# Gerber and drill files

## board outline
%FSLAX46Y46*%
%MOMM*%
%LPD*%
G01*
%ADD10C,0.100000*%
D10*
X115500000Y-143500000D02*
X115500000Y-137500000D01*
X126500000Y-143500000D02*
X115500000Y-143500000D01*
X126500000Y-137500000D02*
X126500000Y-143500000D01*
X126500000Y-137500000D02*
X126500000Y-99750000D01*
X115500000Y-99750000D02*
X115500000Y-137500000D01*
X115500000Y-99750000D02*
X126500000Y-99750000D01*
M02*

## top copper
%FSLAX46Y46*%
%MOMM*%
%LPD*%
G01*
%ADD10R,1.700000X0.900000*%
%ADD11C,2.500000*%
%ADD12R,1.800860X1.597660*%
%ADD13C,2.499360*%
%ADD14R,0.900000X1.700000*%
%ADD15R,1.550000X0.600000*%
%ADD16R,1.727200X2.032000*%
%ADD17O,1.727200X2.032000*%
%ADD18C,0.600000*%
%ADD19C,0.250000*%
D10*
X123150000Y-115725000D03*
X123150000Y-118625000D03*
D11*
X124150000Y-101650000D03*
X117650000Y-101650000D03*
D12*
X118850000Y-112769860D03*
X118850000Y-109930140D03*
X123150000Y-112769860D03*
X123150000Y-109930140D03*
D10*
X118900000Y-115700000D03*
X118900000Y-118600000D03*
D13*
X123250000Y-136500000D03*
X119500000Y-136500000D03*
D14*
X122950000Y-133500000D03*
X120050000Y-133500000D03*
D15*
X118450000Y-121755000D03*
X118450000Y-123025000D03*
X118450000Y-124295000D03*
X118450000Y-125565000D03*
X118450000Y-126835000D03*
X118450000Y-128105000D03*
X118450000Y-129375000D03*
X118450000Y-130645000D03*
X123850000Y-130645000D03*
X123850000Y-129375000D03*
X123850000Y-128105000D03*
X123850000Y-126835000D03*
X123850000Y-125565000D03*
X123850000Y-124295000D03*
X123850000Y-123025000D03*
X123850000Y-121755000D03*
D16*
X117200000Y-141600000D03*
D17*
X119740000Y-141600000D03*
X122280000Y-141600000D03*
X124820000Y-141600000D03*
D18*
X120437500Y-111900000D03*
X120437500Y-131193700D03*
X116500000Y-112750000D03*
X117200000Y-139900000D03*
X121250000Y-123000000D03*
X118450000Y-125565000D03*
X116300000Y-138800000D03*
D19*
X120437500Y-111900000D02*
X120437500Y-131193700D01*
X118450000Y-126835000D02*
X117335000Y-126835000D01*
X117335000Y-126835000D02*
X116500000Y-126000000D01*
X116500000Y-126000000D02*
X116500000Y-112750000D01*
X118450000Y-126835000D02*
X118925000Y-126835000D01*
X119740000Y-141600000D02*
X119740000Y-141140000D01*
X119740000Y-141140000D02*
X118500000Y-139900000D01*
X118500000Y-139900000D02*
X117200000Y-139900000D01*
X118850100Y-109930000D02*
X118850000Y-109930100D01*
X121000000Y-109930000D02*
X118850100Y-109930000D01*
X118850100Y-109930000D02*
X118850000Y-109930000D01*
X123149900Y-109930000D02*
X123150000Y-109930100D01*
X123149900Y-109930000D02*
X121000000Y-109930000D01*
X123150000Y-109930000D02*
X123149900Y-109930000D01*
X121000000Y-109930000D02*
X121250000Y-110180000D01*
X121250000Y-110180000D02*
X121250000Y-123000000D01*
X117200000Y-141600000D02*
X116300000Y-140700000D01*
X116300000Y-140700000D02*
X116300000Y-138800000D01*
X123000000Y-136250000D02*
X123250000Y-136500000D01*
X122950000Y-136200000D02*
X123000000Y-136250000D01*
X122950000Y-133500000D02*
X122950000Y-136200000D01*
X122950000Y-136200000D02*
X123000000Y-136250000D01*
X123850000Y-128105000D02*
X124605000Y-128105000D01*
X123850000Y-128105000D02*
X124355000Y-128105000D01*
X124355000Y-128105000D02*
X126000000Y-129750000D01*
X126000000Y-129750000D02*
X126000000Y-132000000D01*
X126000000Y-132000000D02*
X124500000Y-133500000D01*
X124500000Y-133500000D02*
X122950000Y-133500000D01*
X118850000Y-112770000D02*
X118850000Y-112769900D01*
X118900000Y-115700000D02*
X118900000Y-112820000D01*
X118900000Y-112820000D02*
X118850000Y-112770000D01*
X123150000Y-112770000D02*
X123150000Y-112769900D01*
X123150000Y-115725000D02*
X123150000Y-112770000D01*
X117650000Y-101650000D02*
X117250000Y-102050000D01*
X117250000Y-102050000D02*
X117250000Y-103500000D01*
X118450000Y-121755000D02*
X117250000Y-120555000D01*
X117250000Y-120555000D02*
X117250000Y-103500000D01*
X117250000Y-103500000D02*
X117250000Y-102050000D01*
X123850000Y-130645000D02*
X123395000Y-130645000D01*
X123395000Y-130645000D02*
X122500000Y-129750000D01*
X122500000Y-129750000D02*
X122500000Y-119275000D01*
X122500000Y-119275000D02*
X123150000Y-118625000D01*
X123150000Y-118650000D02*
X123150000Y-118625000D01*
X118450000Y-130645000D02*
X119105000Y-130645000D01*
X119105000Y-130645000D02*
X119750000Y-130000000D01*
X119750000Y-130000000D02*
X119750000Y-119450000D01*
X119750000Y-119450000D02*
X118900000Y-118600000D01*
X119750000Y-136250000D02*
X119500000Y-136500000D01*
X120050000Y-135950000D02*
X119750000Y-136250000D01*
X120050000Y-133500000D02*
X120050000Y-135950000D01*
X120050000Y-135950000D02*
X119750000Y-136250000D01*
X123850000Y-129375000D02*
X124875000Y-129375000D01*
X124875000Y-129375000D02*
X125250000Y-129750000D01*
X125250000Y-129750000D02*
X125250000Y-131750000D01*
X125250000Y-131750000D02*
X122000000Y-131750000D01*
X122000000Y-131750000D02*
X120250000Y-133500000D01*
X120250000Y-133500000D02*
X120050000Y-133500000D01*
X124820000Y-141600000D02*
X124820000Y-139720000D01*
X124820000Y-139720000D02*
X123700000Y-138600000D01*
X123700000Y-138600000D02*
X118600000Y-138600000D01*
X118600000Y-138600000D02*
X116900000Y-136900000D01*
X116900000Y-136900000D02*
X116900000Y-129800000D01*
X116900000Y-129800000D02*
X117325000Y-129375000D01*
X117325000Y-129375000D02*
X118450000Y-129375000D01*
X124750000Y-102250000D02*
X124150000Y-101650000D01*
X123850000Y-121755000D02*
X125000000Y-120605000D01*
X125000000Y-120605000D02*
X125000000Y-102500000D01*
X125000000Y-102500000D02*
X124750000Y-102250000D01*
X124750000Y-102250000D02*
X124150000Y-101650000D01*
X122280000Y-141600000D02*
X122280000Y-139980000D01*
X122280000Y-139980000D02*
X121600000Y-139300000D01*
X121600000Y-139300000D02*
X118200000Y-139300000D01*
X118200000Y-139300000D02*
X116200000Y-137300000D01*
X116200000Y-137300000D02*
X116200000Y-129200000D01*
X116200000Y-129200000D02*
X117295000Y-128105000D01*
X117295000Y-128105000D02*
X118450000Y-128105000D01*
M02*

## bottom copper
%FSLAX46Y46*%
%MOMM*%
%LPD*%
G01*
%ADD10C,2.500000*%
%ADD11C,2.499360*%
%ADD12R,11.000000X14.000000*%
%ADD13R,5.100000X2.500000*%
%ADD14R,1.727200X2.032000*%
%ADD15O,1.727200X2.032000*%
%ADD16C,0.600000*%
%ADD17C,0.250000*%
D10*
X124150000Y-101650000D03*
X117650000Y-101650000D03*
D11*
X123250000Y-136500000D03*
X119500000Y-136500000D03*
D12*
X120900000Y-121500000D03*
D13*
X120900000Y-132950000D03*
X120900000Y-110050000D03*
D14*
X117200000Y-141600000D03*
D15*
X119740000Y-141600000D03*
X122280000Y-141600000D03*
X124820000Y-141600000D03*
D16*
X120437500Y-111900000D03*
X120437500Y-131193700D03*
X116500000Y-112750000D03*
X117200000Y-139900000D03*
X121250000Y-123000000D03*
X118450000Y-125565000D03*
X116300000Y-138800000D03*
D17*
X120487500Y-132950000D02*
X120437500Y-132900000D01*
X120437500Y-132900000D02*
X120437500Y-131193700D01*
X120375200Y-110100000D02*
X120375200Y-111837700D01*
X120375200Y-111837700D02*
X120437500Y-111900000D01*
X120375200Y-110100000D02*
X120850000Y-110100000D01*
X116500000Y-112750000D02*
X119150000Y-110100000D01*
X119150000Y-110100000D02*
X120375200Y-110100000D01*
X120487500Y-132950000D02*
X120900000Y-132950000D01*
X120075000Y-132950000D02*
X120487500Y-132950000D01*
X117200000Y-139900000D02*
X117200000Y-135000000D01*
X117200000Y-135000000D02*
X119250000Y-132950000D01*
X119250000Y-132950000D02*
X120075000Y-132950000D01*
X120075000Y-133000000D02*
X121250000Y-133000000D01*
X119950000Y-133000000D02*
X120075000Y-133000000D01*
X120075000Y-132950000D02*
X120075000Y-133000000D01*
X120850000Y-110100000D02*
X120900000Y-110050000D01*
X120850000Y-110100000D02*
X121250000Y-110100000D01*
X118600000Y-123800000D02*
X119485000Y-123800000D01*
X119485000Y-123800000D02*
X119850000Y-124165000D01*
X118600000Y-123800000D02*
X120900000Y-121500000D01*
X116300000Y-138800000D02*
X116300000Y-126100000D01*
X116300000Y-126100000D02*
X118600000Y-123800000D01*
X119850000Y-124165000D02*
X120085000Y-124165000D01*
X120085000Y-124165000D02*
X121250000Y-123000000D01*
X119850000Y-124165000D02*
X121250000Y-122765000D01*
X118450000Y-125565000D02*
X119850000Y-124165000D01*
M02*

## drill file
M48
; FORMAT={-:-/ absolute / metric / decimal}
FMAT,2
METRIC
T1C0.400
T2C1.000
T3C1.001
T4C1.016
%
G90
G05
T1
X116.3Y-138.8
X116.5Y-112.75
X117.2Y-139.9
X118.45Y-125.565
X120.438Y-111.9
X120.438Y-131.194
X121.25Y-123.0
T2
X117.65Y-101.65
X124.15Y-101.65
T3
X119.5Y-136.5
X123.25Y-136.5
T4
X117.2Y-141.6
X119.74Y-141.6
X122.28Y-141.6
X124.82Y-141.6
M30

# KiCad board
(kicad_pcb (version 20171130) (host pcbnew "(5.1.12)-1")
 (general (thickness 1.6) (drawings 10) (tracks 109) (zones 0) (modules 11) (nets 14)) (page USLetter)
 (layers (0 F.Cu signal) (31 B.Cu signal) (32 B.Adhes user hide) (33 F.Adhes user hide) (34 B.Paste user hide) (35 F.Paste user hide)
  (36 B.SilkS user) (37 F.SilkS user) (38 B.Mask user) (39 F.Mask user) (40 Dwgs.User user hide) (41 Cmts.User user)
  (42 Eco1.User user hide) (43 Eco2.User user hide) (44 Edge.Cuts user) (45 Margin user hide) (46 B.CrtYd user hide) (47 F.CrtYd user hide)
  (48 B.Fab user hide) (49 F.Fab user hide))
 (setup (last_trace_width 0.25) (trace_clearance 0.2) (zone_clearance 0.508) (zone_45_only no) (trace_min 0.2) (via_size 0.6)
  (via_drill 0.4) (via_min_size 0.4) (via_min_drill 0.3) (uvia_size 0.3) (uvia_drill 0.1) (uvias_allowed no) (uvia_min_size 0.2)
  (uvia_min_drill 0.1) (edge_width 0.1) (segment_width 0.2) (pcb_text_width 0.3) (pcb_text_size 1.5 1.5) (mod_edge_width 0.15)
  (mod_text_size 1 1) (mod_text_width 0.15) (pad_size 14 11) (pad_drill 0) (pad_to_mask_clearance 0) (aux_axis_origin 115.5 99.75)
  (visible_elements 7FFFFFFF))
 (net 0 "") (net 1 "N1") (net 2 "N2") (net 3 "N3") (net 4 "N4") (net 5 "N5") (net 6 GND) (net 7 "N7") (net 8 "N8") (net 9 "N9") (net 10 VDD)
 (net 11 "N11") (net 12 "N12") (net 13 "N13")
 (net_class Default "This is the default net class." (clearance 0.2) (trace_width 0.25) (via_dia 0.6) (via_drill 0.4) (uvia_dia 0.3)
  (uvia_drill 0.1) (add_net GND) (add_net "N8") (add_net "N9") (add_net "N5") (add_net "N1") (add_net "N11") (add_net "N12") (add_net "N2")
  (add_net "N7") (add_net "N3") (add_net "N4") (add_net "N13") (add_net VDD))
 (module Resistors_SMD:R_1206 (layer F.Cu) (at 123.15 117.175 270)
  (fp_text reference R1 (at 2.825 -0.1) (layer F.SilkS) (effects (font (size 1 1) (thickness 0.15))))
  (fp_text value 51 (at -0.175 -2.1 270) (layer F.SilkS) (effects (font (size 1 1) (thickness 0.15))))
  (pad 1 smd rect (at -1.45 0 270) (size 0.9 1.7) (layers F.Cu F.Paste F.Mask) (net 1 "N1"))
  (pad 2 smd rect (at 1.45 0 270) (size 0.9 1.7) (layers F.Cu F.Paste F.Mask) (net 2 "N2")))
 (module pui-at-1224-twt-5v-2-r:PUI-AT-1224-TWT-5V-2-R (layer F.Cu) (at 120.9 101.65 180)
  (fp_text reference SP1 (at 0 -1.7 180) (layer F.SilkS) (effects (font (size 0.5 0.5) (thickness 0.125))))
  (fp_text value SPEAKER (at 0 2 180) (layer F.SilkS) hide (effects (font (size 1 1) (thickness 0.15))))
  (pad 1 thru_hole circle (at -3.25 0 180) (size 2.5 2.5) (drill 1) (layers *.Cu *.Mask F.SilkS) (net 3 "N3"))
  (pad 2 thru_hole circle (at 3.25 0 180) (size 2.5 2.5) (drill 1) (layers *.Cu *.Mask F.SilkS) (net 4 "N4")))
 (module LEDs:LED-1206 (layer F.Cu) (at 118.85 111.35 270)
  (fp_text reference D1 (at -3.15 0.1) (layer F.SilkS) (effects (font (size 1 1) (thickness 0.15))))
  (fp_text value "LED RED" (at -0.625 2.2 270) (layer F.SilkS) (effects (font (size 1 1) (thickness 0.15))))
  (pad 2 smd rect (at 1.41986 0 90) (size 1.59766 1.80086) (layers F.Cu F.Paste F.Mask) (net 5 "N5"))
  (pad 1 smd rect (at -1.41986 0 90) (size 1.59766 1.80086) (layers F.Cu F.Paste F.Mask) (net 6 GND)))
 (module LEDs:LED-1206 (layer F.Cu) (at 123.15 111.35 270)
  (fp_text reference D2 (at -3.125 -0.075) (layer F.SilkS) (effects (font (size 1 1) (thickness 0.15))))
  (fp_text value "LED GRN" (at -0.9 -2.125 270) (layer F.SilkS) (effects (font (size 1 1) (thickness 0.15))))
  (pad 2 smd rect (at 1.41986 0 90) (size 1.59766 1.80086) (layers F.Cu F.Paste F.Mask) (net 1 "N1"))
  (pad 1 smd rect (at -1.41986 0 90) (size 1.59766 1.80086) (layers F.Cu F.Paste F.Mask) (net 6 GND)))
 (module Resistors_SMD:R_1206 (layer F.Cu) (at 118.9 117.15 270)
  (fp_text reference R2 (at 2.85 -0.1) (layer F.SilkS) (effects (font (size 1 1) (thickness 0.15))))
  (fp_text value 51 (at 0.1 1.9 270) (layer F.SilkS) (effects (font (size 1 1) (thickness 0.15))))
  (pad 1 smd rect (at -1.45 0 270) (size 0.9 1.7) (layers F.Cu F.Paste F.Mask) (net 5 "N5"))
  (pad 2 smd rect (at 1.45 0 270) (size 0.9 1.7) (layers F.Cu F.Paste F.Mask) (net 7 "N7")))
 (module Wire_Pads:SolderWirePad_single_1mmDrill (layer F.Cu) (at 123.25 136.5)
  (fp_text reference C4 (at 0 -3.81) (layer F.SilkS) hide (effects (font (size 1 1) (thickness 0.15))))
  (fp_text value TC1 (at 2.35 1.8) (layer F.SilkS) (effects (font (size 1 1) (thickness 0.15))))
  (pad 1 thru_hole circle (at 0 0) (size 2.49936 2.49936) (drill 1.00076) (layers *.Cu *.Mask F.SilkS) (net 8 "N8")))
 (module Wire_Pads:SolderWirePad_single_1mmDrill (layer F.Cu) (at 119.5 136.5)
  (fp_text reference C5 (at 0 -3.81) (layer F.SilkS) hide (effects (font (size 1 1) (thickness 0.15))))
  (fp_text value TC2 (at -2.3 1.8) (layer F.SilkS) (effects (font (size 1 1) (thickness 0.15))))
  (pad 1 thru_hole circle (at 0 0) (size 2.49936 2.49936) (drill 1.00076) (layers *.Cu *.Mask F.SilkS) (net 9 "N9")))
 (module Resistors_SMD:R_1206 (layer F.Cu) (at 121.5 133.5 180)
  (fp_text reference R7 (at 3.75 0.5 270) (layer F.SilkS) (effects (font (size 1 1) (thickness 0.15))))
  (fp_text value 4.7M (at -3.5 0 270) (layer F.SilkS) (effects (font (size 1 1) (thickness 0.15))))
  (pad 1 smd rect (at -1.45 0 180) (size 0.9 1.7) (layers F.Cu F.Paste F.Mask) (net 8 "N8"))
  (pad 2 smd rect (at 1.45 0 180) (size 0.9 1.7) (layers F.Cu F.Paste F.Mask) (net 9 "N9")))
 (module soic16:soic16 (layer F.Cu) (at 121.15 126.2) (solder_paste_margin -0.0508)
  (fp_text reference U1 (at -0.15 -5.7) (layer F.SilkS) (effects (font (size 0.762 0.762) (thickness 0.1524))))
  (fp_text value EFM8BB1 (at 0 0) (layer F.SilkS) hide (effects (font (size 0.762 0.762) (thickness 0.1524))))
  (pad 1 smd rect (at -2.7 -4.445) (size 1.55 0.6) (layers F.Cu F.Paste F.Mask) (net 4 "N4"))
  (pad 2 smd rect (at -2.7 -3.175) (size 1.55 0.6) (layers F.Cu F.Paste F.Mask))
  (pad 3 smd rect (at -2.7 -1.905) (size 1.55 0.6) (layers F.Cu F.Paste F.Mask))
  (pad 4 smd rect (at -2.7 -0.635) (size 1.55 0.6) (layers F.Cu F.Paste F.Mask) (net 6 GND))
  (pad 5 smd rect (at -2.7 0.635) (size 1.55 0.6) (layers F.Cu F.Paste F.Mask) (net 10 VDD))
  (pad 6 smd rect (at -2.7 1.905) (size 1.55 0.6) (layers F.Cu F.Paste F.Mask) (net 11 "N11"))
  (pad 7 smd rect (at -2.7 3.175) (size 1.55 0.6) (layers F.Cu F.Paste F.Mask) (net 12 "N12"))
  (pad 8 smd rect (at -2.7 4.445) (size 1.55 0.6) (layers F.Cu F.Paste F.Mask) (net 7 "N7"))
  (pad 9 smd rect (at 2.7 4.445) (size 1.55 0.6) (layers F.Cu F.Paste F.Mask) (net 2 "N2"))
  (pad 10 smd rect (at 2.7 3.175) (size 1.55 0.6) (layers F.Cu F.Paste F.Mask) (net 9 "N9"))
  (pad 11 smd rect (at 2.7 1.905) (size 1.55 0.6) (layers F.Cu F.Paste F.Mask) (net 8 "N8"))
  (pad 12 smd rect (at 2.7 0.635) (size 1.55 0.6) (layers F.Cu F.Paste F.Mask))
  (pad 13 smd rect (at 2.7 -0.635) (size 1.55 0.6) (layers F.Cu F.Paste F.Mask) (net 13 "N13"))
  (pad 14 smd rect (at 2.7 -1.905) (size 1.55 0.6) (layers F.Cu F.Paste F.Mask))
  (pad 15 smd rect (at 2.7 -3.175) (size 1.55 0.6) (layers F.Cu F.Paste F.Mask))
  (pad 16 smd rect (at 2.7 -4.445) (size 1.55 0.6) (layers F.Cu F.Paste F.Mask) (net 3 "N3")))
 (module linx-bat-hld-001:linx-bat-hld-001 (layer B.Cu) (at 120.9 121.5 90)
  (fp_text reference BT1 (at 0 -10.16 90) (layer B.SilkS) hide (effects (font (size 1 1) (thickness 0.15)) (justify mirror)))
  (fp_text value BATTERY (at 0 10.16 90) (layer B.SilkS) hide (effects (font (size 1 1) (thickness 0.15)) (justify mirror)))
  (pad 2 smd rect (at 0 0 90) (size 14 11) (layers B.Cu B.Paste B.Mask) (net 6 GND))
  (pad 1 smd rect (at -11.45 0 90) (size 2.5 5.1) (layers B.Cu B.Paste B.Mask) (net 10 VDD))
  (pad 1 smd rect (at 11.45 0 90) (size 2.5 5.1) (layers B.Cu B.Paste B.Mask) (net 10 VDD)))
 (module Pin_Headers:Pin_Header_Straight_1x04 (layer F.Cu) (at 117.2 141.6 90)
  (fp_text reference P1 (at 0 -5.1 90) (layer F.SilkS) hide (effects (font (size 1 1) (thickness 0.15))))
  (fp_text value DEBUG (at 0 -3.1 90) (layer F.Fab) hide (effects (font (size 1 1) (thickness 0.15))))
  (pad 1 thru_hole rect (at 0 0 90) (size 2.032 1.7272) (drill 1.016) (layers *.Cu *.Mask F.SilkS) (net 6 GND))
  (pad 2 thru_hole oval (at 0 2.54 90) (size 2.032 1.7272) (drill 1.016) (layers *.Cu *.Mask F.SilkS) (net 10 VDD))
  (pad 3 thru_hole oval (at 0 5.08 90) (size 2.032 1.7272) (drill 1.016) (layers *.Cu *.Mask F.SilkS) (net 11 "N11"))
  (pad 4 thru_hole oval (at 0 7.62 90) (size 2.032 1.7272) (drill 1.016) (layers *.Cu *.Mask F.SilkS) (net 12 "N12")))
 (gr_line (start 115.5 143.5) (end 115.5 137.5) (angle 90) (layer Edge.Cuts) (width 0.1))
 (gr_line (start 126.5 143.5) (end 115.5 143.5) (angle 90) (layer Edge.Cuts) (width 0.1))
 (gr_line (start 126.5 137.5) (end 126.5 143.5) (angle 90) (layer Edge.Cuts) (width 0.1))
 (gr_line (start 126.5 137.5) (end 126.5 99.75) (angle 90) (layer Edge.Cuts) (width 0.1))
 (gr_line (start 115.5 99.75) (end 115.5 137.5) (angle 90) (layer Edge.Cuts) (width 0.1))
 (gr_line (start 115.5 99.75) (end 126.5 99.75) (angle 90) (layer Edge.Cuts) (width 0.1))
 (segment (start 120.4375 111.9) (end 120.4375 131.1937) (width 0.25) (layer F.Cu) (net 10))
 (segment (start 120.4875 132.95) (end 120.4375 132.9) (width 0.25) (layer B.Cu) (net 10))
 (segment (start 120.4375 132.9) (end 120.4375 131.1937) (width 0.25) (layer B.Cu) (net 10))
 (segment (start 120.3752 110.1) (end 120.3752 111.8377) (width 0.25) (layer B.Cu) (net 10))
 (segment (start 120.3752 111.8377) (end 120.4375 111.9) (width 0.25) (layer B.Cu) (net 10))
 (segment (start 120.3752 110.1) (end 120.85 110.1) (width 0.25) (layer B.Cu) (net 10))
 (segment (start 116.5 112.75) (end 119.15 110.1) (width 0.25) (layer B.Cu) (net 10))
 (segment (start 119.15 110.1) (end 120.3752 110.1) (width 0.25) (layer B.Cu) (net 10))
 (segment (start 120.4875 132.95) (end 120.9 132.95) (width 0.25) (layer B.Cu) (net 10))
 (segment (start 120.075 132.95) (end 120.4875 132.95) (width 0.25) (layer B.Cu) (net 10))
 (segment (start 117.2 139.9) (end 117.2 135) (width 0.25) (layer B.Cu) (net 10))
 (segment (start 117.2 135) (end 119.25 132.95) (width 0.25) (layer B.Cu) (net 10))
 (segment (start 119.25 132.95) (end 120.075 132.95) (width 0.25) (layer B.Cu) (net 10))
 (segment (start 120.075 133) (end 121.25 133) (width 0.25) (layer B.Cu) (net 10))
 (segment (start 119.95 133) (end 120.075 133) (width 0.25) (layer B.Cu) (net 10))
 (segment (start 120.075 132.95) (end 120.075 133) (width 0.25) (layer B.Cu) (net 10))
 (segment (start 120.85 110.1) (end 120.9 110.05) (width 0.25) (layer B.Cu) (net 10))
 (segment (start 120.85 110.1) (end 121.25 110.1) (width 0.25) (layer B.Cu) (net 10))
 (segment (start 118.45 126.835) (end 117.335 126.835) (width 0.25) (layer F.Cu) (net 10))
 (segment (start 117.335 126.835) (end 116.5 126) (width 0.25) (layer F.Cu) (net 10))
 (segment (start 116.5 126) (end 116.5 112.75) (width 0.25) (layer F.Cu) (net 10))
 (segment (start 118.45 126.835) (end 118.925 126.835) (width 0.25) (layer F.Cu) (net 10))
 (segment (start 119.74 141.6) (end 119.74 141.14) (width 0.25) (layer F.Cu) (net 10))
 (segment (start 119.74 141.14) (end 118.5 139.9) (width 0.25) (layer F.Cu) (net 10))
 (segment (start 118.5 139.9) (end 117.2 139.9) (width 0.25) (layer F.Cu) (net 10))
 (via (at 120.4375 111.9) (size 0.6) (layers F.Cu B.Cu) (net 10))
 (via (at 120.4375 131.1937) (size 0.6) (layers F.Cu B.Cu) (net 10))
 (via (at 116.5 112.75) (size 0.6) (layers F.Cu B.Cu) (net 10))
 (via (at 117.2 139.9) (size 0.6) (layers F.Cu B.Cu) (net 10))
 (segment (start 118.8501 109.93) (end 118.85 109.9301) (width 0.25) (layer F.Cu) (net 6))
 (segment (start 121 109.93) (end 118.8501 109.93) (width 0.25) (layer F.Cu) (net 6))
 (segment (start 118.8501 109.93) (end 118.85 109.93) (width 0.25) (layer F.Cu) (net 6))
 (segment (start 118.6 123.8) (end 119.485 123.8) (width 0.25) (layer B.Cu) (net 6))
 (segment (start 119.485 123.8) (end 119.85 124.165) (width 0.25) (layer B.Cu) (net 6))
 (segment (start 118.6 123.8) (end 120.9 121.5) (width 0.25) (layer B.Cu) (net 6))
 (segment (start 116.3 138.8) (end 116.3 126.1) (width 0.25) (layer B.Cu) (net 6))
 (segment (start 116.3 126.1) (end 118.6 123.8) (width 0.25) (layer B.Cu) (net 6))
 (segment (start 119.85 124.165) (end 120.085 124.165) (width 0.25) (layer B.Cu) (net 6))
 (segment (start 120.085 124.165) (end 121.25 123) (width 0.25) (layer B.Cu) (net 6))
 (segment (start 119.85 124.165) (end 121.25 122.765) (width 0.25) (layer B.Cu) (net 6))
 (segment (start 118.45 125.565) (end 119.85 124.165) (width 0.25) (layer B.Cu) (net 6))
 (segment (start 123.1499 109.93) (end 123.15 109.9301) (width 0.25) (layer F.Cu) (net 6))
 (segment (start 123.1499 109.93) (end 121 109.93) (width 0.25) (layer F.Cu) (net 6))
 (segment (start 123.15 109.93) (end 123.1499 109.93) (width 0.25) (layer F.Cu) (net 6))
 (segment (start 121 109.93) (end 121.25 110.18) (width 0.25) (layer F.Cu) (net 6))
 (segment (start 121.25 110.18) (end 121.25 123) (width 0.25) (layer F.Cu) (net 6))
 (segment (start 117.2 141.6) (end 116.3 140.7) (width 0.25) (layer F.Cu) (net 6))
 (segment (start 116.3 140.7) (end 116.3 138.8) (width 0.25) (layer F.Cu) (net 6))
 (via (at 121.25 123) (size 0.6) (layers F.Cu B.Cu) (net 6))
 (via (at 118.45 125.565) (size 0.6) (layers F.Cu B.Cu) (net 6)) (via (at 116.3 138.8) (size 0.6) (layers F.Cu B.Cu) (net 6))
 (segment (start 123 136.25) (end 123.25 136.5) (width 0.25) (layer F.Cu) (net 8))
 (segment (start 122.95 136.2) (end 123 136.25) (width 0.25) (layer F.Cu) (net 8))
 (segment (start 122.95 133.5) (end 122.95 136.2) (width 0.25) (layer F.Cu) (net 8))
 (segment (start 122.95 136.2) (end 123 136.25) (width 0.25) (layer F.Cu) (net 8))
 (segment (start 123.85 128.105) (end 124.605 128.105) (width 0.25) (layer F.Cu) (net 8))
 (segment (start 123.85 128.105) (end 124.355 128.105) (width 0.25) (layer F.Cu) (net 8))
 (segment (start 124.355 128.105) (end 126 129.75) (width 0.25) (layer F.Cu) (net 8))
 (segment (start 126 129.75) (end 126 132) (width 0.25) (layer F.Cu) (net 8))
 (segment (start 126 132) (end 124.5 133.5) (width 0.25) (layer F.Cu) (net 8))
 (segment (start 124.5 133.5) (end 122.95 133.5) (width 0.25) (layer F.Cu) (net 8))
 (segment (start 118.85 112.77) (end 118.85 112.7699) (width 0.25) (layer F.Cu) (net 5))
 (segment (start 118.9 115.7) (end 118.9 112.82) (width 0.25) (layer F.Cu) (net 5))
 (segment (start 118.9 112.82) (end 118.85 112.77) (width 0.25) (layer F.Cu) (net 5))
 (segment (start 123.15 112.77) (end 123.15 112.7699) (width 0.25) (layer F.Cu) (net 1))
 (segment (start 123.15 115.725) (end 123.15 112.77) (width 0.25) (layer F.Cu) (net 1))
 (segment (start 117.65 101.65) (end 117.25 102.05) (width 0.25) (layer F.Cu) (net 4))
 (segment (start 117.25 102.05) (end 117.25 103.5) (width 0.25) (layer F.Cu) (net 4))
 (segment (start 118.45 121.755) (end 117.25 120.555) (width 0.25) (layer F.Cu) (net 4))
 (segment (start 117.25 120.555) (end 117.25 103.5) (width 0.25) (layer F.Cu) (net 4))
 (segment (start 117.25 103.5) (end 117.25 102.05) (width 0.25) (layer F.Cu) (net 4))
 (segment (start 123.85 130.645) (end 123.395 130.645) (width 0.25) (layer F.Cu) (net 2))
 (segment (start 123.395 130.645) (end 122.5 129.75) (width 0.25) (layer F.Cu) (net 2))
 (segment (start 122.5 129.75) (end 122.5 119.275) (width 0.25) (layer F.Cu) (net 2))
 (segment (start 122.5 119.275) (end 123.15 118.625) (width 0.25) (layer F.Cu) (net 2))
 (segment (start 123.15 118.65) (end 123.15 118.625) (width 0.25) (layer F.Cu) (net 2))
 (segment (start 118.45 130.645) (end 119.105 130.645) (width 0.25) (layer F.Cu) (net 7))
 (segment (start 119.105 130.645) (end 119.75 130) (width 0.25) (layer F.Cu) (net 7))
 (segment (start 119.75 130) (end 119.75 119.45) (width 0.25) (layer F.Cu) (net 7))
 (segment (start 119.75 119.45) (end 118.9 118.6) (width 0.25) (layer F.Cu) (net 7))
 (segment (start 119.75 136.25) (end 119.5 136.5) (width 0.25) (layer F.Cu) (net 9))
 (segment (start 120.05 135.95) (end 119.75 136.25) (width 0.25) (layer F.Cu) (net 9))
 (segment (start 120.05 133.5) (end 120.05 135.95) (width 0.25) (layer F.Cu) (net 9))
 (segment (start 120.05 135.95) (end 119.75 136.25) (width 0.25) (layer F.Cu) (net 9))
 (segment (start 123.85 129.375) (end 124.875 129.375) (width 0.25) (layer F.Cu) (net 9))
 (segment (start 124.875 129.375) (end 125.25 129.75) (width 0.25) (layer F.Cu) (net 9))
 (segment (start 125.25 129.75) (end 125.25 131.75) (width 0.25) (layer F.Cu) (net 9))
 (segment (start 125.25 131.75) (end 122 131.75) (width 0.25) (layer F.Cu) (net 9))
 (segment (start 122 131.75) (end 120.25 133.5) (width 0.25) (layer F.Cu) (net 9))
 (segment (start 120.25 133.5) (end 120.05 133.5) (width 0.25) (layer F.Cu) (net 9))
 (segment (start 124.82 141.6) (end 124.82 139.72) (width 0.25) (layer F.Cu) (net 12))
 (segment (start 124.82 139.72) (end 123.7 138.6) (width 0.25) (layer F.Cu) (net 12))
 (segment (start 123.7 138.6) (end 118.6 138.6) (width 0.25) (layer F.Cu) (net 12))
 (segment (start 118.6 138.6) (end 116.9 136.9) (width 0.25) (layer F.Cu) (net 12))
 (segment (start 116.9 136.9) (end 116.9 129.8) (width 0.25) (layer F.Cu) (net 12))
 (segment (start 116.9 129.8) (end 117.325 129.375) (width 0.25) (layer F.Cu) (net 12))
 (segment (start 117.325 129.375) (end 118.45 129.375) (width 0.25) (layer F.Cu) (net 12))
 (segment (start 124.75 102.25) (end 124.15 101.65) (width 0.25) (layer F.Cu) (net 3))
 (segment (start 123.85 121.755) (end 125 120.605) (width 0.25) (layer F.Cu) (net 3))
 (segment (start 125 120.605) (end 125 102.5) (width 0.25) (layer F.Cu) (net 3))
 (segment (start 125 102.5) (end 124.75 102.25) (width 0.25) (layer F.Cu) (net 3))
 (segment (start 124.75 102.25) (end 124.15 101.65) (width 0.25) (layer F.Cu) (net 3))
 (segment (start 122.28 141.6) (end 122.28 139.98) (width 0.25) (layer F.Cu) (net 11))
 (segment (start 122.28 139.98) (end 121.6 139.3) (width 0.25) (layer F.Cu) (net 11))
 (segment (start 121.6 139.3) (end 118.2 139.3) (width 0.25) (layer F.Cu) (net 11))
 (segment (start 118.2 139.3) (end 116.2 137.3) (width 0.25) (layer F.Cu) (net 11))
 (segment (start 116.2 137.3) (end 116.2 129.2) (width 0.25) (layer F.Cu) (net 11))
 (segment (start 116.2 129.2) (end 117.295 128.105) (width 0.25) (layer F.Cu) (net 11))
 (segment (start 117.295 128.105) (end 118.45 128.105) (width 0.25) (layer F.Cu) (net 11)))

